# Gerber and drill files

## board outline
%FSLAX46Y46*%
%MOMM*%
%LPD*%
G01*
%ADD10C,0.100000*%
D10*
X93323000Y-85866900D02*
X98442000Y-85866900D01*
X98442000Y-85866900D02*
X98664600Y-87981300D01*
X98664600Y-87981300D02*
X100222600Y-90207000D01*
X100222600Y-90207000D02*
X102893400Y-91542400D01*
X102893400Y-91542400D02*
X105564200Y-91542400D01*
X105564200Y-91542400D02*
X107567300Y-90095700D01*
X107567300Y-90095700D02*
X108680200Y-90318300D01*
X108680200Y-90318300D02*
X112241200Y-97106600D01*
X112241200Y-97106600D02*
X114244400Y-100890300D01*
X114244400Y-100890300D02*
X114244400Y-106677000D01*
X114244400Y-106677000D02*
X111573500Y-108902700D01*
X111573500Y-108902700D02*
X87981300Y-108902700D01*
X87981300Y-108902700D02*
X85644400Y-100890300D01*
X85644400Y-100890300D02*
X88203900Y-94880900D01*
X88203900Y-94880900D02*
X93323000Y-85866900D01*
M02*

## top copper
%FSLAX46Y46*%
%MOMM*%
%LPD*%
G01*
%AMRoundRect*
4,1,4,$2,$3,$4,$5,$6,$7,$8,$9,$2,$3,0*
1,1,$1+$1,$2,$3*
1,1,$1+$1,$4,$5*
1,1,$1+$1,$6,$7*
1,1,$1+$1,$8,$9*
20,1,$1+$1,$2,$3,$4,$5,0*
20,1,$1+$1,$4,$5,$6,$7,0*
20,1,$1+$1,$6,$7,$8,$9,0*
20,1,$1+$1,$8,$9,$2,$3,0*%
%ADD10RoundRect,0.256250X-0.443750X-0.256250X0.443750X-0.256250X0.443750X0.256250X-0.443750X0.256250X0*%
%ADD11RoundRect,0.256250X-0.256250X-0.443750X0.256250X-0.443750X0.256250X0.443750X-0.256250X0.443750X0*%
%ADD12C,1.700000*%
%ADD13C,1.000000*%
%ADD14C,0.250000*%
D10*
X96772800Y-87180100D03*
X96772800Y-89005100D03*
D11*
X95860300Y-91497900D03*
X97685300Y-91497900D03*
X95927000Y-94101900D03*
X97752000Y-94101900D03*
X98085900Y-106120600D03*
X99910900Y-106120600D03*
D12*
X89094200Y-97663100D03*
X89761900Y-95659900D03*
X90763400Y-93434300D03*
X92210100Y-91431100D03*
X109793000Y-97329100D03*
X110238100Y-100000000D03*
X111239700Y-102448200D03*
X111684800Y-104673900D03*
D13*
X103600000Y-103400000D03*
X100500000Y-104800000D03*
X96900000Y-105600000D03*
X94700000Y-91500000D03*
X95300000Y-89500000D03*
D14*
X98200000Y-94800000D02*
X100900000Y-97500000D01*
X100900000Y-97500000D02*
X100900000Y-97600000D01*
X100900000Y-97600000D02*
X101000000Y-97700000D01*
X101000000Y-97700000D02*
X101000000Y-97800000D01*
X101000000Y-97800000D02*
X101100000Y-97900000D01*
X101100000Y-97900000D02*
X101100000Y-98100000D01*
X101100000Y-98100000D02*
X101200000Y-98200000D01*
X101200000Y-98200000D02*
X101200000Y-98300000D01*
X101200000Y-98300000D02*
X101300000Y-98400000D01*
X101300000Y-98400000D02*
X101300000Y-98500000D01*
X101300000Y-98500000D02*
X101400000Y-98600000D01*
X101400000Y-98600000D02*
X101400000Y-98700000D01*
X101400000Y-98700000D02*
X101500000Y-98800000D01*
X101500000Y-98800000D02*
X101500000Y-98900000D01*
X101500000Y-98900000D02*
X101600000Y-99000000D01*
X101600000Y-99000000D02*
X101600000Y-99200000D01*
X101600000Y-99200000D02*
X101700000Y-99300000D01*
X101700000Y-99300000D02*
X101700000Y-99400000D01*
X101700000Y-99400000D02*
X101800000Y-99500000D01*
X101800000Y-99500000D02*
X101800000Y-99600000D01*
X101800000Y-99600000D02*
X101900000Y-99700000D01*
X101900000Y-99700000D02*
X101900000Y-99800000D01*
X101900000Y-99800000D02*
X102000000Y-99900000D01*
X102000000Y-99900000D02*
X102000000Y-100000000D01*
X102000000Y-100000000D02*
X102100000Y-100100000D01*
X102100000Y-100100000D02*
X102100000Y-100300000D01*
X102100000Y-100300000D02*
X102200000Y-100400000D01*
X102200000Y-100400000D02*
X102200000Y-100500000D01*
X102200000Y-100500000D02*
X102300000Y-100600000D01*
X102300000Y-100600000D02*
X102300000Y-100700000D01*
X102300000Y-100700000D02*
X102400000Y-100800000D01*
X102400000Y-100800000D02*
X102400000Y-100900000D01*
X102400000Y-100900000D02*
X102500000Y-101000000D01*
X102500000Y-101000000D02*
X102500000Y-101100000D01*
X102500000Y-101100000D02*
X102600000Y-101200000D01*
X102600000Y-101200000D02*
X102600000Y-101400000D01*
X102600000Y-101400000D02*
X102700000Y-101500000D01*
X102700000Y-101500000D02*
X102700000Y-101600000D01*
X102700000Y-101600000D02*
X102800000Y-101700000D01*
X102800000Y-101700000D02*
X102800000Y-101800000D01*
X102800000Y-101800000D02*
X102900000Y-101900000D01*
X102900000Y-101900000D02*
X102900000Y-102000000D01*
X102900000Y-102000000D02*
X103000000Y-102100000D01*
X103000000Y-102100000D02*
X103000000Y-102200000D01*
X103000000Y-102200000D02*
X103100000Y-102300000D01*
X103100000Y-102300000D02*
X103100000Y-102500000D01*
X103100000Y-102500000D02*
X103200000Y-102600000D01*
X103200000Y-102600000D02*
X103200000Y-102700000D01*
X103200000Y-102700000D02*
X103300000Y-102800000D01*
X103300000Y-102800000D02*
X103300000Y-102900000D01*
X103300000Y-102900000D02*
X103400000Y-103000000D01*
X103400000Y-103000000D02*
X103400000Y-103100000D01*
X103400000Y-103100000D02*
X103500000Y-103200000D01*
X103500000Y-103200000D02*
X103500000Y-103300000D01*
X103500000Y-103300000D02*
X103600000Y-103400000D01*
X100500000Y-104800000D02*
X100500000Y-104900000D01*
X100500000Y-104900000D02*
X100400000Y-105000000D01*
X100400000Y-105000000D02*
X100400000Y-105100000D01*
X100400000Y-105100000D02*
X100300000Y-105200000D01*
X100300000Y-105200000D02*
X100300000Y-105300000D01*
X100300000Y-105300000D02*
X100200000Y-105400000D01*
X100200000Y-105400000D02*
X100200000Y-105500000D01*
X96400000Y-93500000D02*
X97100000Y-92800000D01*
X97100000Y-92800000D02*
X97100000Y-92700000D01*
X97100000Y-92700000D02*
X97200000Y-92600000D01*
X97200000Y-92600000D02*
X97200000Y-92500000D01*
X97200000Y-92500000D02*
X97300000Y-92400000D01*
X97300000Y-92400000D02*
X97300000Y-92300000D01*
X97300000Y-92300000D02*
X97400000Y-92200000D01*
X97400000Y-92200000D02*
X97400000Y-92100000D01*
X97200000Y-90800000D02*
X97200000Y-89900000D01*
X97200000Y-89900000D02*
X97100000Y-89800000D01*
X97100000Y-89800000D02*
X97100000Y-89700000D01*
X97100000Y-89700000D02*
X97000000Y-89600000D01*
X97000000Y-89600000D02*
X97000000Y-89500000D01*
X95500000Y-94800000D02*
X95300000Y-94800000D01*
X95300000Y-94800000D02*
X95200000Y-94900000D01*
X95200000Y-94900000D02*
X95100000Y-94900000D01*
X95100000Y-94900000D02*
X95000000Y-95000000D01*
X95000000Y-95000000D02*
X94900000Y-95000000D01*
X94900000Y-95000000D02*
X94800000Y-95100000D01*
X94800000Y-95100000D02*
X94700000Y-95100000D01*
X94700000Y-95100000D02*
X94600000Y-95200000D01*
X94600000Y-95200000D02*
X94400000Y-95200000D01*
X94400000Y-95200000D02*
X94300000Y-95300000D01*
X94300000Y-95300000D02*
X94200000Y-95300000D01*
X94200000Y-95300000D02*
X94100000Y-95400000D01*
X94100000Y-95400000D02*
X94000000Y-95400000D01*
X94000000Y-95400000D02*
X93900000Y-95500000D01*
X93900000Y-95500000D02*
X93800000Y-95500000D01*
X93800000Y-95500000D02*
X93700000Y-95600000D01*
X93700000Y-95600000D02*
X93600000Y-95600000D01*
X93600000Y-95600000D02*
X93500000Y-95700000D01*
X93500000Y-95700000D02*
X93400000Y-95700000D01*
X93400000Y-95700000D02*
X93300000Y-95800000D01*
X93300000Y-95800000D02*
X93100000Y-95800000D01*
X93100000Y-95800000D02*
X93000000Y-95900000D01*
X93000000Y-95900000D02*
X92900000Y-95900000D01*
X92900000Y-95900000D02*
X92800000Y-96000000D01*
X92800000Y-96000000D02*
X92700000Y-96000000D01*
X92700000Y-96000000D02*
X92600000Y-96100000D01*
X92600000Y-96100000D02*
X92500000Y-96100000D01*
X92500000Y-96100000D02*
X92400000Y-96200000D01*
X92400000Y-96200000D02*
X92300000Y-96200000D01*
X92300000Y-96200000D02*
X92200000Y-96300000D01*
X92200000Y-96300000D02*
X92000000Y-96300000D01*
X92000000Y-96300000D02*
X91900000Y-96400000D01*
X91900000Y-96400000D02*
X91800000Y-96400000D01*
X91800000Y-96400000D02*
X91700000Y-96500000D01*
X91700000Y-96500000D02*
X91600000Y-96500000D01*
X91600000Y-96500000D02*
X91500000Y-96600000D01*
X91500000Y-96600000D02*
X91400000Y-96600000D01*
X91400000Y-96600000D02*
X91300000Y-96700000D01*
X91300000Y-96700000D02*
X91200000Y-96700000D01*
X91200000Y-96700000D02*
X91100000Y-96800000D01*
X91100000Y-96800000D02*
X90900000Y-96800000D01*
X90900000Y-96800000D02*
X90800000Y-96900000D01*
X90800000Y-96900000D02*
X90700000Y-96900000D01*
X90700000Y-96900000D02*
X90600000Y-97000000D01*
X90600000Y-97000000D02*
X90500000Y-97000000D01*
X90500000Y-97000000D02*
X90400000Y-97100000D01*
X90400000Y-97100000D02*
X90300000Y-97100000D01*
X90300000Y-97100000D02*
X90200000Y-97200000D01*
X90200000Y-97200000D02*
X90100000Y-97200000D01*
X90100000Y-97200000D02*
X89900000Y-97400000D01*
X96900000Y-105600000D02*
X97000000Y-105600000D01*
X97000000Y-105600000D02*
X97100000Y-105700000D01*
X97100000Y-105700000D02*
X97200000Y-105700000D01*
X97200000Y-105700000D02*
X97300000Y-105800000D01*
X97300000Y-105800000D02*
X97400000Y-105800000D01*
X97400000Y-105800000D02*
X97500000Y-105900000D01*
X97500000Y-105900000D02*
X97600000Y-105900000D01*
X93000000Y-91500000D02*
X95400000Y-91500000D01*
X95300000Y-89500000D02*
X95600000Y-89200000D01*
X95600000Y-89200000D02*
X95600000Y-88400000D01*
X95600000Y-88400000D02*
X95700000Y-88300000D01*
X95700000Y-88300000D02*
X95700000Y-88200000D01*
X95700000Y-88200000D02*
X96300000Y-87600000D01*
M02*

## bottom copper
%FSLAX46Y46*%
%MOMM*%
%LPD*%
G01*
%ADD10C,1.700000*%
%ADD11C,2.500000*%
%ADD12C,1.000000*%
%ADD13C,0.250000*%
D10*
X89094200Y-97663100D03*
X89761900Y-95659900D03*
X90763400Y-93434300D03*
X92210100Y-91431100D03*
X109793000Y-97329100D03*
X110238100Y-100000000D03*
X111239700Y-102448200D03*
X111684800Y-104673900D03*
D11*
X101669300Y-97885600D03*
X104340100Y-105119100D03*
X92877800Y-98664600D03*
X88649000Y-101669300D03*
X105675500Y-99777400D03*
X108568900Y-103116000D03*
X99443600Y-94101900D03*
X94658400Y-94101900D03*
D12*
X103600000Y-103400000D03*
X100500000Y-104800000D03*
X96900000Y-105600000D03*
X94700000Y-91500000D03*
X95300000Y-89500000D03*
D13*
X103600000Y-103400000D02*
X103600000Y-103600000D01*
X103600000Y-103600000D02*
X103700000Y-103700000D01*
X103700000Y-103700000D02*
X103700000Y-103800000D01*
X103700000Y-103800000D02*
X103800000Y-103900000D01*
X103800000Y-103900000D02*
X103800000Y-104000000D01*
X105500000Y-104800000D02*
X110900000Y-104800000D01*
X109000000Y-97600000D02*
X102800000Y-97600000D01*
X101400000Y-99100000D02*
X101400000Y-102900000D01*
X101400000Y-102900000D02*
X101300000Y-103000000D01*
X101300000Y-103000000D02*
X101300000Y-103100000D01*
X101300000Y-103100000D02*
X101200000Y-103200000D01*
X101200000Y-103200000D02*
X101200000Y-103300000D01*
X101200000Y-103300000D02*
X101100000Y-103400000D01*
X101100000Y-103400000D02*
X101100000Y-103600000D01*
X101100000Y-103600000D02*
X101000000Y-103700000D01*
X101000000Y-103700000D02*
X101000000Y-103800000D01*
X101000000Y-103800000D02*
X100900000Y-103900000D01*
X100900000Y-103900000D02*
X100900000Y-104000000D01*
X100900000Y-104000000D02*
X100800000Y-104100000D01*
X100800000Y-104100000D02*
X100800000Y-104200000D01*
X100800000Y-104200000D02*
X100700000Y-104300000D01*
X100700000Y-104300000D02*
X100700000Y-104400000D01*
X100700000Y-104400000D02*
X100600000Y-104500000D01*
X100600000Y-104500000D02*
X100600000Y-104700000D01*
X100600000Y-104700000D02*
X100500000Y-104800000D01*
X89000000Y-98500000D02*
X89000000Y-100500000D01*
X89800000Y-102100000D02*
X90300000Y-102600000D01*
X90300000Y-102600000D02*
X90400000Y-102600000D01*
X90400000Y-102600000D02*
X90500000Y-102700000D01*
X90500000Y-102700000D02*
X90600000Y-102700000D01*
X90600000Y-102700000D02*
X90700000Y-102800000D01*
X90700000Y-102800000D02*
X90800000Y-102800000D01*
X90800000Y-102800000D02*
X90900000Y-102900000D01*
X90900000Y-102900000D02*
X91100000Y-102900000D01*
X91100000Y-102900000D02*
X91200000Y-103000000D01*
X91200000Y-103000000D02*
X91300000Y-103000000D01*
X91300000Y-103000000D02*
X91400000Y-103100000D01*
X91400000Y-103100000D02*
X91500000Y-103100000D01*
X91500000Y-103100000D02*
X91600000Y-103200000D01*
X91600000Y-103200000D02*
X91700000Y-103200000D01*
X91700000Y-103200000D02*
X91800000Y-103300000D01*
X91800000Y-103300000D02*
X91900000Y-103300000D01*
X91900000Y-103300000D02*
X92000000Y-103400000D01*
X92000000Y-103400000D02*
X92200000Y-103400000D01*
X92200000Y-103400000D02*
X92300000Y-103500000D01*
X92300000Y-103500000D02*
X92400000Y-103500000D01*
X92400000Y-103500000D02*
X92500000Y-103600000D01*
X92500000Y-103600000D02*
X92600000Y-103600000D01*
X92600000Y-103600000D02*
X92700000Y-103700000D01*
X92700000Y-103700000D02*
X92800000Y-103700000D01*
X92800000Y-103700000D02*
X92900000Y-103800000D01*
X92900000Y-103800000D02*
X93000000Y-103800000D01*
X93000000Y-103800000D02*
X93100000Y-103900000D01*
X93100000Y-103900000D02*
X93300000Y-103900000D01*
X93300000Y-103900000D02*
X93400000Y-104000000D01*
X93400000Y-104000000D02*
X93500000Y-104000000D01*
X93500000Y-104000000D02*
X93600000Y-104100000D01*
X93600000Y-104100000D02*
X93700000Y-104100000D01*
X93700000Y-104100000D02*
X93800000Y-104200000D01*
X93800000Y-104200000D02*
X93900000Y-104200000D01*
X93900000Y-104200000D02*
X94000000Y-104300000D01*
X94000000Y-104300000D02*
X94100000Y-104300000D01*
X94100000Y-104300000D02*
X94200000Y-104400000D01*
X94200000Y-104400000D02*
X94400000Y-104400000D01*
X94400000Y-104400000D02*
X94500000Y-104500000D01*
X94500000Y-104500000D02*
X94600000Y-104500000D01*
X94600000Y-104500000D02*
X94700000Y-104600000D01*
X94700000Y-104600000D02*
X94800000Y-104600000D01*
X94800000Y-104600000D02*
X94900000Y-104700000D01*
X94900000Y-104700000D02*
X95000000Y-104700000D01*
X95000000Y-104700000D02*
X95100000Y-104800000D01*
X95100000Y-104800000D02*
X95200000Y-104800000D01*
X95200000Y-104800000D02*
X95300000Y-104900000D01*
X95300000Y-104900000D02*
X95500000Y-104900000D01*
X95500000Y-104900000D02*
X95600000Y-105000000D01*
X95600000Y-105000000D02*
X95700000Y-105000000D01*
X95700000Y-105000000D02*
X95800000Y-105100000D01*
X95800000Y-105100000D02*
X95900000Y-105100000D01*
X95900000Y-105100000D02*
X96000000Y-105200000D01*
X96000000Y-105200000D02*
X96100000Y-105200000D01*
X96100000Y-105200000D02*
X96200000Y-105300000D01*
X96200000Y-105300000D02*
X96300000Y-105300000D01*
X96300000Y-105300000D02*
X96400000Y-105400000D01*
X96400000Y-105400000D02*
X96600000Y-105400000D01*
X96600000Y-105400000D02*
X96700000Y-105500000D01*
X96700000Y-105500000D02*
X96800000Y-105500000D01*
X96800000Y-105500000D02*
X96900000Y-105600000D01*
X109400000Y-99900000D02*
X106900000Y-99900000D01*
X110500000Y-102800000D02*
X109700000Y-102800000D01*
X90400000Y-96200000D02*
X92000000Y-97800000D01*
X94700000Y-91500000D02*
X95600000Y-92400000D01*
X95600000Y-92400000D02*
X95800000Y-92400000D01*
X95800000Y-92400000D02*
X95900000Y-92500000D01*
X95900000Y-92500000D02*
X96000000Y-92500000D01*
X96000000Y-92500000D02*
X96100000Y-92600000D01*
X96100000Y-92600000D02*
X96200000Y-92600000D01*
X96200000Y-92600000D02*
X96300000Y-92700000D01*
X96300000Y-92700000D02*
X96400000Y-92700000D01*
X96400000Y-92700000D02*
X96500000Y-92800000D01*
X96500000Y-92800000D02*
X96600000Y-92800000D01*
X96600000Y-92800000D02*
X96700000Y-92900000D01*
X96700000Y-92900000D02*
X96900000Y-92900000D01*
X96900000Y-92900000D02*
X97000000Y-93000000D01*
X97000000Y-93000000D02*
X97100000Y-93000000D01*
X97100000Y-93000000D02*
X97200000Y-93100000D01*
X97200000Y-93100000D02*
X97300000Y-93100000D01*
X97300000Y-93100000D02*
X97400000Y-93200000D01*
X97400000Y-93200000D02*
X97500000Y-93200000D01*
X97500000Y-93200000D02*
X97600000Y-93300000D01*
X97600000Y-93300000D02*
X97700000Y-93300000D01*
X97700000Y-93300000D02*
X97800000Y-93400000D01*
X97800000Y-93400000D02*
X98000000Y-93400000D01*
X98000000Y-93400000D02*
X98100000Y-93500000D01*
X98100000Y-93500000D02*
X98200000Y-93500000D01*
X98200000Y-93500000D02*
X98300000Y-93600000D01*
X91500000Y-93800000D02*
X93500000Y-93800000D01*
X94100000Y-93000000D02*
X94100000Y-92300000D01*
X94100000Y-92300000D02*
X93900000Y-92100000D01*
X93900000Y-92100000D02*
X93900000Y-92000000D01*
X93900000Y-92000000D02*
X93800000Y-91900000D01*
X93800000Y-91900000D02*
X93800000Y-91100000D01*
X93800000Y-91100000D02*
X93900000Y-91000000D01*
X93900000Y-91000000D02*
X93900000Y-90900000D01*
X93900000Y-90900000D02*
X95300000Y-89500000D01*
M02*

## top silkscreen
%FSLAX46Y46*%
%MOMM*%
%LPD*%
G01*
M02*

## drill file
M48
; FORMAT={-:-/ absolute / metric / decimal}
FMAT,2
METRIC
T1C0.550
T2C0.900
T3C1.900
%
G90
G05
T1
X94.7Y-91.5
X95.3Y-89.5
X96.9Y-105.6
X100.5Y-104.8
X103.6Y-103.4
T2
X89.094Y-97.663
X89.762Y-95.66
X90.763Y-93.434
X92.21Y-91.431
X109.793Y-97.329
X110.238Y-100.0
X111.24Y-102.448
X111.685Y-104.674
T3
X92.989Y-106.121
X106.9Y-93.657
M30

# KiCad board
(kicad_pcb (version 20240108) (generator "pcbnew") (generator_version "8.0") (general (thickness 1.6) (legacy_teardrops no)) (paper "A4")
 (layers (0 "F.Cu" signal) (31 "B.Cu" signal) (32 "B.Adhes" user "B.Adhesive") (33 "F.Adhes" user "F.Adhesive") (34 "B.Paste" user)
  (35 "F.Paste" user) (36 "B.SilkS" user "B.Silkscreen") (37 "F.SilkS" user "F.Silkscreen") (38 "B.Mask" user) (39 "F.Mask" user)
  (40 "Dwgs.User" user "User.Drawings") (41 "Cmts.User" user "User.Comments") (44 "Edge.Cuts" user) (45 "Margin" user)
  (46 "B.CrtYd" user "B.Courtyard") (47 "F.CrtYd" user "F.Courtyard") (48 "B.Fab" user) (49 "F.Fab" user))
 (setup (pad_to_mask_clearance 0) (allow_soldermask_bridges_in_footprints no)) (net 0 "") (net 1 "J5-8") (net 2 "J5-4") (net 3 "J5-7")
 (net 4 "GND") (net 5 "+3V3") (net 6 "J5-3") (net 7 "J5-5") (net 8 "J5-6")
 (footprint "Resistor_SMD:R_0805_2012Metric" (layer "F.Cu") (at 96.7728 88.0926)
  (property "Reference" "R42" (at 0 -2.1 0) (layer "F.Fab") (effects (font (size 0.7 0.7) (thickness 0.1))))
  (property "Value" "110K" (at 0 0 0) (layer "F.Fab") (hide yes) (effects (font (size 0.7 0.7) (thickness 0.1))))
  (pad "1" smd roundrect (at 0 -0.9125) (size 1.4 1.025) (layers "F.Cu" "F.Mask" "F.Paste") (roundrect_rratio 0.25) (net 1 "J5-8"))
  (pad "2" smd roundrect (at 0 0.9125) (size 1.4 1.025) (layers "F.Cu" "F.Mask" "F.Paste") (roundrect_rratio 0.25) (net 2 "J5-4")))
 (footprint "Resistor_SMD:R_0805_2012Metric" (layer "F.Cu") (at 96.7728 91.4979)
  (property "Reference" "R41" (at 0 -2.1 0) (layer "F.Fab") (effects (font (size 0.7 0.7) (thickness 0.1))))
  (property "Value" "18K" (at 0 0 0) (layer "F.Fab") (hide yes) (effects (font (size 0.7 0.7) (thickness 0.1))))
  (pad "1" smd roundrect (at -0.9125 0) (size 1.025 1.4) (layers "F.Cu" "F.Mask" "F.Paste") (roundrect_rratio 0.25) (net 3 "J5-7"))
  (pad "2" smd roundrect (at 0.9125 0) (size 1.025 1.4) (layers "F.Cu" "F.Mask" "F.Paste") (roundrect_rratio 0.25) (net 2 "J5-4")))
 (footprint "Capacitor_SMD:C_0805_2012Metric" (layer "F.Cu") (at 96.8395 94.1019)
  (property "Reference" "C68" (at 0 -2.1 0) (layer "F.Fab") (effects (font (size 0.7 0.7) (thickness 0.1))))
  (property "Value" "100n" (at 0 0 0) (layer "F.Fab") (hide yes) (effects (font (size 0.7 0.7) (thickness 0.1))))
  (pad "1" smd roundrect (at -0.9125 0) (size 1.025 1.4) (layers "F.Cu" "F.Mask" "F.Paste") (roundrect_rratio 0.25) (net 2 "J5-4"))
  (pad "2" smd roundrect (at 0.9125 0) (size 1.025 1.4) (layers "F.Cu" "F.Mask" "F.Paste") (roundrect_rratio 0.25) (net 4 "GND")))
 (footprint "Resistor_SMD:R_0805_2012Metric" (layer "F.Cu") (at 98.9984 106.1206)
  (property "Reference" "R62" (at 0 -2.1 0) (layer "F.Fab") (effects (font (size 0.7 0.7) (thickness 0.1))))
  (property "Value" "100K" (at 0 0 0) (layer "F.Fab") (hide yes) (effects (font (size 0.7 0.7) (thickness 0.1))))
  (pad "1" smd roundrect (at -0.9125 0) (size 1.025 1.4) (layers "F.Cu" "F.Mask" "F.Paste") (roundrect_rratio 0.25) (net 2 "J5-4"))
  (pad "2" smd roundrect (at 0.9125 0) (size 1.025 1.4) (layers "F.Cu" "F.Mask" "F.Paste") (roundrect_rratio 0.25) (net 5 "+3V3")))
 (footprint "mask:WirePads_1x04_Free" (layer "F.Cu") (at 90.4574 94.5471)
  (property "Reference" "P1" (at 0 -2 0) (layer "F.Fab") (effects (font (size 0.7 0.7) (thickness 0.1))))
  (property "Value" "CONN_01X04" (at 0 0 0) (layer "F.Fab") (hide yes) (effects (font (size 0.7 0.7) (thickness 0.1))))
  (pad "1" thru_hole circle (at -1.3632 3.116) (size 1.7 1.7) (drill 0.9) (layers "*.Cu" "*.Mask") (remove_unused_layers no) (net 2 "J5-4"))
  (pad "2" thru_hole circle (at -0.6955 1.1128) (size 1.7 1.7) (drill 0.9) (layers "*.Cu" "*.Mask") (remove_unused_layers no) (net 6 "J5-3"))
  (pad "3" thru_hole circle (at 0.306 -1.1128) (size 1.7 1.7) (drill 0.9) (layers "*.Cu" "*.Mask") (remove_unused_layers no) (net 1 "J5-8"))
  (pad "4" thru_hole circle (at 1.7527 -3.116) (size 1.7 1.7) (drill 0.9) (layers "*.Cu" "*.Mask") (remove_unused_layers no) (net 3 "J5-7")))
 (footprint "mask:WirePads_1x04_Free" (layer "F.Cu") (at 110.7389 101.1128)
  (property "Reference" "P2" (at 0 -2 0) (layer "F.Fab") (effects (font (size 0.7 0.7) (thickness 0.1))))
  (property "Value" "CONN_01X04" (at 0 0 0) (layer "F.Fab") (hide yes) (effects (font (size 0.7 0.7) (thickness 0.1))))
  (pad "1" thru_hole circle (at -0.9459 -3.7837) (size 1.7 1.7) (drill 0.9) (layers "*.Cu" "*.Mask") (remove_unused_layers no)
   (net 5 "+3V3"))
  (pad "2" thru_hole circle (at -0.5008 -1.1128) (size 1.7 1.7) (drill 0.9) (layers "*.Cu" "*.Mask") (remove_unused_layers no)
   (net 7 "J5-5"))
  (pad "3" thru_hole circle (at 0.5008 1.3354) (size 1.7 1.7) (drill 0.9) (layers "*.Cu" "*.Mask") (remove_unused_layers no) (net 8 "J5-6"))
  (pad "4" thru_hole circle (at 0.9459 3.5611) (size 1.7 1.7) (drill 0.9) (layers "*.Cu" "*.Mask") (remove_unused_layers no) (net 4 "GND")))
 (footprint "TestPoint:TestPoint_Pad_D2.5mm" (layer "B.Cu") (at 101.6693 97.8856)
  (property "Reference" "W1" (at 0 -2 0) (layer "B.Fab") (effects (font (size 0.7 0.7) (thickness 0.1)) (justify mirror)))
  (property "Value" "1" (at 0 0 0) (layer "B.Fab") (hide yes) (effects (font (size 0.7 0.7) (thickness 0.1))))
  (pad "1" smd circle (at 0 0) (size 2.5 2.5) (layers "B.Cu" "B.Mask") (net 5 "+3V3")))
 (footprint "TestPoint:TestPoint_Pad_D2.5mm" (layer "B.Cu") (at 104.3401 105.1191)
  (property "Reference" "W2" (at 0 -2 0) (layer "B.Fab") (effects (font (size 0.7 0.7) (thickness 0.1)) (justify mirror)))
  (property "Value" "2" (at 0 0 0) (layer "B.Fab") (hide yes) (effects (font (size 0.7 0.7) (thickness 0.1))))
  (pad "1" smd circle (at 0 0) (size 2.5 2.5) (layers "B.Cu" "B.Mask") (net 4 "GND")))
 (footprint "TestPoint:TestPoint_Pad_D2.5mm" (layer "B.Cu") (at 92.8778 98.6646)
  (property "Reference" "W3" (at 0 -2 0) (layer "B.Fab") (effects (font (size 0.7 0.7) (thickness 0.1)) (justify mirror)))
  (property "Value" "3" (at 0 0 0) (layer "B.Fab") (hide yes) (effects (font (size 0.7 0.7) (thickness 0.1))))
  (pad "1" smd circle (at 0 0) (size 2.5 2.5) (layers "B.Cu" "B.Mask") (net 6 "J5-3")))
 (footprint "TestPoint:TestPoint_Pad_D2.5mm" (layer "B.Cu") (at 88.649 101.6693)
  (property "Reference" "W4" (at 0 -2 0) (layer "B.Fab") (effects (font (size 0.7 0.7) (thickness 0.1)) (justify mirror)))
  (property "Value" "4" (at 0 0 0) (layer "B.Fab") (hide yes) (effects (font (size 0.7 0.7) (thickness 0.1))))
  (pad "1" smd circle (at 0 0) (size 2.5 2.5) (layers "B.Cu" "B.Mask") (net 2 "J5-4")))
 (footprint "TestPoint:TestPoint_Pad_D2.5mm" (layer "B.Cu") (at 105.6755 99.7774)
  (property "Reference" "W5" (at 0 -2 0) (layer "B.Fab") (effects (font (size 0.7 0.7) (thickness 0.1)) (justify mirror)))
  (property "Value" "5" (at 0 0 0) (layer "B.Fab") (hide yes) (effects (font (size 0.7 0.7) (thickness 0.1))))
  (pad "1" smd circle (at 0 0) (size 2.5 2.5) (layers "B.Cu" "B.Mask") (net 7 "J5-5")))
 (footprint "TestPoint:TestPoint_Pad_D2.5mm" (layer "B.Cu") (at 108.5689 103.116)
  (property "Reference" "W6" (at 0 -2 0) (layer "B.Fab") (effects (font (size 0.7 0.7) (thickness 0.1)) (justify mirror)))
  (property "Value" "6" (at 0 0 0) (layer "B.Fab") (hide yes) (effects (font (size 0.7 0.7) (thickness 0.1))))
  (pad "1" smd circle (at 0 0) (size 2.5 2.5) (layers "B.Cu" "B.Mask") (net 8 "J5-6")))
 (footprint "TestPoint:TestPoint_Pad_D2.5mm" (layer "B.Cu") (at 99.4436 94.1019)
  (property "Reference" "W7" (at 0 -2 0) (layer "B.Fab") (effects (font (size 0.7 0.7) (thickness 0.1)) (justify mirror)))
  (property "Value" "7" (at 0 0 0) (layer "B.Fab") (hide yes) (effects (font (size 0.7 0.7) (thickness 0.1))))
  (pad "1" smd circle (at 0 0) (size 2.5 2.5) (layers "B.Cu" "B.Mask") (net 3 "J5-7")))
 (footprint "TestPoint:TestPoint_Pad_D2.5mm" (layer "B.Cu") (at 94.6584 94.1019)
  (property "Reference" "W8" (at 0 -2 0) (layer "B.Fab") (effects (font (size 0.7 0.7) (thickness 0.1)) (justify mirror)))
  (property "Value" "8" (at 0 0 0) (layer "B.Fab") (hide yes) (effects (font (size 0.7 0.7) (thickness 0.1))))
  (pad "1" smd circle (at 0 0) (size 2.5 2.5) (layers "B.Cu" "B.Mask") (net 1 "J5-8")))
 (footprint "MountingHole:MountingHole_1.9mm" (layer "F.Cu") (at 92.9891 106.1206)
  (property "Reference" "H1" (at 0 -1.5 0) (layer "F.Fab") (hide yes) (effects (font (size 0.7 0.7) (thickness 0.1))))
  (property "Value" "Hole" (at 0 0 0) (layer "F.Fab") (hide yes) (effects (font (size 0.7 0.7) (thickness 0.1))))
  (pad "" np_thru_hole circle (at 0 0) (size 1.9 1.9) (drill 1.9) (layers "*.Cu" "*.Mask")))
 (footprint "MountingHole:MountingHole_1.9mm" (layer "F.Cu") (at 106.8996 93.6568)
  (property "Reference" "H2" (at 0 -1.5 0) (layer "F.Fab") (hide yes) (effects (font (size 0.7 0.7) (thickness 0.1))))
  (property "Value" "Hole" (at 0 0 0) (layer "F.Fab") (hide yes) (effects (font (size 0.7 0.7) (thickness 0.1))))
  (pad "" np_thru_hole circle (at 0 0) (size 1.9 1.9) (drill 1.9) (layers "*.Cu" "*.Mask")))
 (segment (start 98.2 94.8) (end 100.9 97.5) (width 0.25) (layer "F.Cu") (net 4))
 (segment (start 100.9 97.5) (end 100.9 97.6) (width 0.25) (layer "F.Cu") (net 4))
 (segment (start 100.9 97.6) (end 101 97.7) (width 0.25) (layer "F.Cu") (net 4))
 (segment (start 101 97.7) (end 101 97.8) (width 0.25) (layer "F.Cu") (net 4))
 (segment (start 101 97.8) (end 101.1 97.9) (width 0.25) (layer "F.Cu") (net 4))
 (segment (start 101.1 97.9) (end 101.1 98.1) (width 0.25) (layer "F.Cu") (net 4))
 (segment (start 101.1 98.1) (end 101.2 98.2) (width 0.25) (layer "F.Cu") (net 4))
 (segment (start 101.2 98.2) (end 101.2 98.3) (width 0.25) (layer "F.Cu") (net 4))
 (segment (start 101.2 98.3) (end 101.3 98.4) (width 0.25) (layer "F.Cu") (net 4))
 (segment (start 101.3 98.4) (end 101.3 98.5) (width 0.25) (layer "F.Cu") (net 4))
 (segment (start 101.3 98.5) (end 101.4 98.6) (width 0.25) (layer "F.Cu") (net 4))
 (segment (start 101.4 98.6) (end 101.4 98.7) (width 0.25) (layer "F.Cu") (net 4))
 (segment (start 101.4 98.7) (end 101.5 98.8) (width 0.25) (layer "F.Cu") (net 4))
 (segment (start 101.5 98.8) (end 101.5 98.9) (width 0.25) (layer "F.Cu") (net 4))
 (segment (start 101.5 98.9) (end 101.6 99) (width 0.25) (layer "F.Cu") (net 4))
 (segment (start 101.6 99) (end 101.6 99.2) (width 0.25) (layer "F.Cu") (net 4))
 (segment (start 101.6 99.2) (end 101.7 99.3) (width 0.25) (layer "F.Cu") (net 4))
 (segment (start 101.7 99.3) (end 101.7 99.4) (width 0.25) (layer "F.Cu") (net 4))
 (segment (start 101.7 99.4) (end 101.8 99.5) (width 0.25) (layer "F.Cu") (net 4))
 (segment (start 101.8 99.5) (end 101.8 99.6) (width 0.25) (layer "F.Cu") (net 4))
 (segment (start 101.8 99.6) (end 101.9 99.7) (width 0.25) (layer "F.Cu") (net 4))
 (segment (start 101.9 99.7) (end 101.9 99.8) (width 0.25) (layer "F.Cu") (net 4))
 (segment (start 101.9 99.8) (end 102 99.9) (width 0.25) (layer "F.Cu") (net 4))
 (segment (start 102 99.9) (end 102 100) (width 0.25) (layer "F.Cu") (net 4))
 (segment (start 102 100) (end 102.1 100.1) (width 0.25) (layer "F.Cu") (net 4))
 (segment (start 102.1 100.1) (end 102.1 100.3) (width 0.25) (layer "F.Cu") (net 4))
 (segment (start 102.1 100.3) (end 102.2 100.4) (width 0.25) (layer "F.Cu") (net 4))
 (segment (start 102.2 100.4) (end 102.2 100.5) (width 0.25) (layer "F.Cu") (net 4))
 (segment (start 102.2 100.5) (end 102.3 100.6) (width 0.25) (layer "F.Cu") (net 4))
 (segment (start 102.3 100.6) (end 102.3 100.7) (width 0.25) (layer "F.Cu") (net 4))
 (segment (start 102.3 100.7) (end 102.4 100.8) (width 0.25) (layer "F.Cu") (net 4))
 (segment (start 102.4 100.8) (end 102.4 100.9) (width 0.25) (layer "F.Cu") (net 4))
 (segment (start 102.4 100.9) (end 102.5 101) (width 0.25) (layer "F.Cu") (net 4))
 (segment (start 102.5 101) (end 102.5 101.1) (width 0.25) (layer "F.Cu") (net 4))
 (segment (start 102.5 101.1) (end 102.6 101.2) (width 0.25) (layer "F.Cu") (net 4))
 (segment (start 102.6 101.2) (end 102.6 101.4) (width 0.25) (layer "F.Cu") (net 4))
 (segment (start 102.6 101.4) (end 102.7 101.5) (width 0.25) (layer "F.Cu") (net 4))
 (segment (start 102.7 101.5) (end 102.7 101.6) (width 0.25) (layer "F.Cu") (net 4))
 (segment (start 102.7 101.6) (end 102.8 101.7) (width 0.25) (layer "F.Cu") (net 4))
 (segment (start 102.8 101.7) (end 102.8 101.8) (width 0.25) (layer "F.Cu") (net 4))
 (segment (start 102.8 101.8) (end 102.9 101.9) (width 0.25) (layer "F.Cu") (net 4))
 (segment (start 102.9 101.9) (end 102.9 102) (width 0.25) (layer "F.Cu") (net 4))
 (segment (start 102.9 102) (end 103 102.1) (width 0.25) (layer "F.Cu") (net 4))
 (segment (start 103 102.1) (end 103 102.2) (width 0.25) (layer "F.Cu") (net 4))
 (segment (start 103 102.2) (end 103.1 102.3) (width 0.25) (layer "F.Cu") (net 4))
 (segment (start 103.1 102.3) (end 103.1 102.5) (width 0.25) (layer "F.Cu") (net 4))
 (segment (start 103.1 102.5) (end 103.2 102.6) (width 0.25) (layer "F.Cu") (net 4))
 (segment (start 103.2 102.6) (end 103.2 102.7) (width 0.25) (layer "F.Cu") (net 4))
 (segment (start 103.2 102.7) (end 103.3 102.8) (width 0.25) (layer "F.Cu") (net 4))
 (segment (start 103.3 102.8) (end 103.3 102.9) (width 0.25) (layer "F.Cu") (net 4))
 (segment (start 103.3 102.9) (end 103.4 103) (width 0.25) (layer "F.Cu") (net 4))
 (segment (start 103.4 103) (end 103.4 103.1) (width 0.25) (layer "F.Cu") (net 4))
 (segment (start 103.4 103.1) (end 103.5 103.2) (width 0.25) (layer "F.Cu") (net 4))
 (segment (start 103.5 103.2) (end 103.5 103.3) (width 0.25) (layer "F.Cu") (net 4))
 (segment (start 103.5 103.3) (end 103.6 103.4) (width 0.25) (layer "F.Cu") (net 4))
 (segment (start 103.6 103.4) (end 103.6 103.6) (width 0.25) (layer "B.Cu") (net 4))
 (segment (start 103.6 103.6) (end 103.7 103.7) (width 0.25) (layer "B.Cu") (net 4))
 (segment (start 103.7 103.7) (end 103.7 103.8) (width 0.25) (layer "B.Cu") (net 4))
 (segment (start 103.7 103.8) (end 103.8 103.9) (width 0.25) (layer "B.Cu") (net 4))
 (segment (start 103.8 103.9) (end 103.8 104) (width 0.25) (layer "B.Cu") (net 4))
 (segment (start 105.5 104.8) (end 110.9 104.8) (width 0.25) (layer "B.Cu") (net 4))
 (via (at 103.6 103.4) (size 1) (drill 0.55) (layers "F.Cu" "B.Cu") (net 4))
 (segment (start 109 97.6) (end 102.8 97.6) (width 0.25) (layer "B.Cu") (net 5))
 (segment (start 101.4 99.1) (end 101.4 102.9) (width 0.25) (layer "B.Cu") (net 5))
 (segment (start 101.4 102.9) (end 101.3 103) (width 0.25) (layer "B.Cu") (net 5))
 (segment (start 101.3 103) (end 101.3 103.1) (width 0.25) (layer "B.Cu") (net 5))
 (segment (start 101.3 103.1) (end 101.2 103.2) (width 0.25) (layer "B.Cu") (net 5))
 (segment (start 101.2 103.2) (end 101.2 103.3) (width 0.25) (layer "B.Cu") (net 5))
 (segment (start 101.2 103.3) (end 101.1 103.4) (width 0.25) (layer "B.Cu") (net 5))
 (segment (start 101.1 103.4) (end 101.1 103.6) (width 0.25) (layer "B.Cu") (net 5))
 (segment (start 101.1 103.6) (end 101 103.7) (width 0.25) (layer "B.Cu") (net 5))
 (segment (start 101 103.7) (end 101 103.8) (width 0.25) (layer "B.Cu") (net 5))
 (segment (start 101 103.8) (end 100.9 103.9) (width 0.25) (layer "B.Cu") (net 5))
 (segment (start 100.9 103.9) (end 100.9 104) (width 0.25) (layer "B.Cu") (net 5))
 (segment (start 100.9 104) (end 100.8 104.1) (width 0.25) (layer "B.Cu") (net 5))
 (segment (start 100.8 104.1) (end 100.8 104.2) (width 0.25) (layer "B.Cu") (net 5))
 (segment (start 100.8 104.2) (end 100.7 104.3) (width 0.25) (layer "B.Cu") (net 5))
 (segment (start 100.7 104.3) (end 100.7 104.4) (width 0.25) (layer "B.Cu") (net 5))
 (segment (start 100.7 104.4) (end 100.6 104.5) (width 0.25) (layer "B.Cu") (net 5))
 (segment (start 100.6 104.5) (end 100.6 104.7) (width 0.25) (layer "B.Cu") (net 5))
 (segment (start 100.6 104.7) (end 100.5 104.8) (width 0.25) (layer "B.Cu") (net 5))
 (segment (start 100.5 104.8) (end 100.5 104.9) (width 0.25) (layer "F.Cu") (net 5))
 (segment (start 100.5 104.9) (end 100.4 105) (width 0.25) (layer "F.Cu") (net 5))
 (segment (start 100.4 105) (end 100.4 105.1) (width 0.25) (layer "F.Cu") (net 5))
 (segment (start 100.4 105.1) (end 100.3 105.2) (width 0.25) (layer "F.Cu") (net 5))
 (segment (start 100.3 105.2) (end 100.3 105.3) (width 0.25) (layer "F.Cu") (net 5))
 (segment (start 100.3 105.3) (end 100.2 105.4) (width 0.25) (layer "F.Cu") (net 5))
 (segment (start 100.2 105.4) (end 100.2 105.5) (width 0.25) (layer "F.Cu") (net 5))
 (via (at 100.5 104.8) (size 1) (drill 0.55) (layers "F.Cu" "B.Cu") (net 5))
 (segment (start 96.4 93.5) (end 97.1 92.8) (width 0.25) (layer "F.Cu") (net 2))
 (segment (start 97.1 92.8) (end 97.1 92.7) (width 0.25) (layer "F.Cu") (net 2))
 (segment (start 97.1 92.7) (end 97.2 92.6) (width 0.25) (layer "F.Cu") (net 2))
 (segment (start 97.2 92.6) (end 97.2 92.5) (width 0.25) (layer "F.Cu") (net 2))
 (segment (start 97.2 92.5) (end 97.3 92.4) (width 0.25) (layer "F.Cu") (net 2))
 (segment (start 97.3 92.4) (end 97.3 92.3) (width 0.25) (layer "F.Cu") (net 2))
 (segment (start 97.3 92.3) (end 97.4 92.2) (width 0.25) (layer "F.Cu") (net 2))
 (segment (start 97.4 92.2) (end 97.4 92.1) (width 0.25) (layer "F.Cu") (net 2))
 (segment (start 97.2 90.8) (end 97.2 89.9) (width 0.25) (layer "F.Cu") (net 2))
 (segment (start 97.2 89.9) (end 97.1 89.8) (width 0.25) (layer "F.Cu") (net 2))
 (segment (start 97.1 89.8) (end 97.1 89.7) (width 0.25) (layer "F.Cu") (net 2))
 (segment (start 97.1 89.7) (end 97 89.6) (width 0.25) (layer "F.Cu") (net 2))
 (segment (start 97 89.6) (end 97 89.5) (width 0.25) (layer "F.Cu") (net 2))
 (segment (start 95.5 94.8) (end 95.3 94.8) (width 0.25) (layer "F.Cu") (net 2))
 (segment (start 95.3 94.8) (end 95.2 94.9) (width 0.25) (layer "F.Cu") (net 2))
 (segment (start 95.2 94.9) (end 95.1 94.9) (width 0.25) (layer "F.Cu") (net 2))
 (segment (start 95.1 94.9) (end 95 95) (width 0.25) (layer "F.Cu") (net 2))
 (segment (start 95 95) (end 94.9 95) (width 0.25) (layer "F.Cu") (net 2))
 (segment (start 94.9 95) (end 94.8 95.1) (width 0.25) (layer "F.Cu") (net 2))
 (segment (start 94.8 95.1) (end 94.7 95.1) (width 0.25) (layer "F.Cu") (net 2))
 (segment (start 94.7 95.1) (end 94.6 95.2) (width 0.25) (layer "F.Cu") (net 2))
 (segment (start 94.6 95.2) (end 94.4 95.2) (width 0.25) (layer "F.Cu") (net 2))
 (segment (start 94.4 95.2) (end 94.3 95.3) (width 0.25) (layer "F.Cu") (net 2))
 (segment (start 94.3 95.3) (end 94.2 95.3) (width 0.25) (layer "F.Cu") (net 2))
 (segment (start 94.2 95.3) (end 94.1 95.4) (width 0.25) (layer "F.Cu") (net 2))
 (segment (start 94.1 95.4) (end 94 95.4) (width 0.25) (layer "F.Cu") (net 2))
 (segment (start 94 95.4) (end 93.9 95.5) (width 0.25) (layer "F.Cu") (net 2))
 (segment (start 93.9 95.5) (end 93.8 95.5) (width 0.25) (layer "F.Cu") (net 2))
 (segment (start 93.8 95.5) (end 93.7 95.6) (width 0.25) (layer "F.Cu") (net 2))
 (segment (start 93.7 95.6) (end 93.6 95.6) (width 0.25) (layer "F.Cu") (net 2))
 (segment (start 93.6 95.6) (end 93.5 95.7) (width 0.25) (layer "F.Cu") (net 2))
 (segment (start 93.5 95.7) (end 93.4 95.7) (width 0.25) (layer "F.Cu") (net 2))
 (segment (start 93.4 95.7) (end 93.3 95.8) (width 0.25) (layer "F.Cu") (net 2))
 (segment (start 93.3 95.8) (end 93.1 95.8) (width 0.25) (layer "F.Cu") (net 2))
 (segment (start 93.1 95.8) (end 93 95.9) (width 0.25) (layer "F.Cu") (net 2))
 (segment (start 93 95.9) (end 92.9 95.9) (width 0.25) (layer "F.Cu") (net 2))
 (segment (start 92.9 95.9) (end 92.8 96) (width 0.25) (layer "F.Cu") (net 2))
 (segment (start 92.8 96) (end 92.7 96) (width 0.25) (layer "F.Cu") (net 2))
 (segment (start 92.7 96) (end 92.6 96.1) (width 0.25) (layer "F.Cu") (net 2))
 (segment (start 92.6 96.1) (end 92.5 96.1) (width 0.25) (layer "F.Cu") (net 2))
 (segment (start 92.5 96.1) (end 92.4 96.2) (width 0.25) (layer "F.Cu") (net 2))
 (segment (start 92.4 96.2) (end 92.3 96.2) (width 0.25) (layer "F.Cu") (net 2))
 (segment (start 92.3 96.2) (end 92.2 96.3) (width 0.25) (layer "F.Cu") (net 2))
 (segment (start 92.2 96.3) (end 92 96.3) (width 0.25) (layer "F.Cu") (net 2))
 (segment (start 92 96.3) (end 91.9 96.4) (width 0.25) (layer "F.Cu") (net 2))
 (segment (start 91.9 96.4) (end 91.8 96.4) (width 0.25) (layer "F.Cu") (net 2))
 (segment (start 91.8 96.4) (end 91.7 96.5) (width 0.25) (layer "F.Cu") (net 2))
 (segment (start 91.7 96.5) (end 91.6 96.5) (width 0.25) (layer "F.Cu") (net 2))
 (segment (start 91.6 96.5) (end 91.5 96.6) (width 0.25) (layer "F.Cu") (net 2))
 (segment (start 91.5 96.6) (end 91.4 96.6) (width 0.25) (layer "F.Cu") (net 2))
 (segment (start 91.4 96.6) (end 91.3 96.7) (width 0.25) (layer "F.Cu") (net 2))
 (segment (start 91.3 96.7) (end 91.2 96.7) (width 0.25) (layer "F.Cu") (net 2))
 (segment (start 91.2 96.7) (end 91.1 96.8) (width 0.25) (layer "F.Cu") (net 2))
 (segment (start 91.1 96.8) (end 90.9 96.8) (width 0.25) (layer "F.Cu") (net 2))
 (segment (start 90.9 96.8) (end 90.8 96.9) (width 0.25) (layer "F.Cu") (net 2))
 (segment (start 90.8 96.9) (end 90.7 96.9) (width 0.25) (layer "F.Cu") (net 2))
 (segment (start 90.7 96.9) (end 90.6 97) (width 0.25) (layer "F.Cu") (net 2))
 (segment (start 90.6 97) (end 90.5 97) (width 0.25) (layer "F.Cu") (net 2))
 (segment (start 90.5 97) (end 90.4 97.1) (width 0.25) (layer "F.Cu") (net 2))
 (segment (start 90.4 97.1) (end 90.3 97.1) (width 0.25) (layer "F.Cu") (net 2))
 (segment (start 90.3 97.1) (end 90.2 97.2) (width 0.25) (layer "F.Cu") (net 2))
 (segment (start 90.2 97.2) (end 90.1 97.2) (width 0.25) (layer "F.Cu") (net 2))
 (segment (start 90.1 97.2) (end 89.9 97.4) (width 0.25) (layer "F.Cu") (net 2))
 (segment (start 89 98.5) (end 89 100.5) (width 0.25) (layer "B.Cu") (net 2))
 (segment (start 89.8 102.1) (end 90.3 102.6) (width 0.25) (layer "B.Cu") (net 2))
 (segment (start 90.3 102.6) (end 90.4 102.6) (width 0.25) (layer "B.Cu") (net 2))
 (segment (start 90.4 102.6) (end 90.5 102.7) (width 0.25) (layer "B.Cu") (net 2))
 (segment (start 90.5 102.7) (end 90.6 102.7) (width 0.25) (layer "B.Cu") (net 2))
 (segment (start 90.6 102.7) (end 90.7 102.8) (width 0.25) (layer "B.Cu") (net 2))
 (segment (start 90.7 102.8) (end 90.8 102.8) (width 0.25) (layer "B.Cu") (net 2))
 (segment (start 90.8 102.8) (end 90.9 102.9) (width 0.25) (layer "B.Cu") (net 2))
 (segment (start 90.9 102.9) (end 91.1 102.9) (width 0.25) (layer "B.Cu") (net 2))
 (segment (start 91.1 102.9) (end 91.2 103) (width 0.25) (layer "B.Cu") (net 2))
 (segment (start 91.2 103) (end 91.3 103) (width 0.25) (layer "B.Cu") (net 2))
 (segment (start 91.3 103) (end 91.4 103.1) (width 0.25) (layer "B.Cu") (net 2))
 (segment (start 91.4 103.1) (end 91.5 103.1) (width 0.25) (layer "B.Cu") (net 2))
 (segment (start 91.5 103.1) (end 91.6 103.2) (width 0.25) (layer "B.Cu") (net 2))
 (segment (start 91.6 103.2) (end 91.7 103.2) (width 0.25) (layer "B.Cu") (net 2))
 (segment (start 91.7 103.2) (end 91.8 103.3) (width 0.25) (layer "B.Cu") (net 2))
 (segment (start 91.8 103.3) (end 91.9 103.3) (width 0.25) (layer "B.Cu") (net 2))
 (segment (start 91.9 103.3) (end 92 103.4) (width 0.25) (layer "B.Cu") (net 2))
 (segment (start 92 103.4) (end 92.2 103.4) (width 0.25) (layer "B.Cu") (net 2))
 (segment (start 92.2 103.4) (end 92.3 103.5) (width 0.25) (layer "B.Cu") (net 2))
 (segment (start 92.3 103.5) (end 92.4 103.5) (width 0.25) (layer "B.Cu") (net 2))
 (segment (start 92.4 103.5) (end 92.5 103.6) (width 0.25) (layer "B.Cu") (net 2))
 (segment (start 92.5 103.6) (end 92.6 103.6) (width 0.25) (layer "B.Cu") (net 2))
 (segment (start 92.6 103.6) (end 92.7 103.7) (width 0.25) (layer "B.Cu") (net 2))
 (segment (start 92.7 103.7) (end 92.8 103.7) (width 0.25) (layer "B.Cu") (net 2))
 (segment (start 92.8 103.7) (end 92.9 103.8) (width 0.25) (layer "B.Cu") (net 2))
 (segment (start 92.9 103.8) (end 93 103.8) (width 0.25) (layer "B.Cu") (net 2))
 (segment (start 93 103.8) (end 93.1 103.9) (width 0.25) (layer "B.Cu") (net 2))
 (segment (start 93.1 103.9) (end 93.3 103.9) (width 0.25) (layer "B.Cu") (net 2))
 (segment (start 93.3 103.9) (end 93.4 104) (width 0.25) (layer "B.Cu") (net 2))
 (segment (start 93.4 104) (end 93.5 104) (width 0.25) (layer "B.Cu") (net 2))
 (segment (start 93.5 104) (end 93.6 104.1) (width 0.25) (layer "B.Cu") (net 2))
 (segment (start 93.6 104.1) (end 93.7 104.1) (width 0.25) (layer "B.Cu") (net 2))
 (segment (start 93.7 104.1) (end 93.8 104.2) (width 0.25) (layer "B.Cu") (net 2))
 (segment (start 93.8 104.2) (end 93.9 104.2) (width 0.25) (layer "B.Cu") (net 2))
 (segment (start 93.9 104.2) (end 94 104.3) (width 0.25) (layer "B.Cu") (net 2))
 (segment (start 94 104.3) (end 94.1 104.3) (width 0.25) (layer "B.Cu") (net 2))
 (segment (start 94.1 104.3) (end 94.2 104.4) (width 0.25) (layer "B.Cu") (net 2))
 (segment (start 94.2 104.4) (end 94.4 104.4) (width 0.25) (layer "B.Cu") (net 2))
 (segment (start 94.4 104.4) (end 94.5 104.5) (width 0.25) (layer "B.Cu") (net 2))
 (segment (start 94.5 104.5) (end 94.6 104.5) (width 0.25) (layer "B.Cu") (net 2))
 (segment (start 94.6 104.5) (end 94.7 104.6) (width 0.25) (layer "B.Cu") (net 2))
 (segment (start 94.7 104.6) (end 94.8 104.6) (width 0.25) (layer "B.Cu") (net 2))
 (segment (start 94.8 104.6) (end 94.9 104.7) (width 0.25) (layer "B.Cu") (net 2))
 (segment (start 94.9 104.7) (end 95 104.7) (width 0.25) (layer "B.Cu") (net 2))
 (segment (start 95 104.7) (end 95.1 104.8) (width 0.25) (layer "B.Cu") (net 2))
 (segment (start 95.1 104.8) (end 95.2 104.8) (width 0.25) (layer "B.Cu") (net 2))
 (segment (start 95.2 104.8) (end 95.3 104.9) (width 0.25) (layer "B.Cu") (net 2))
 (segment (start 95.3 104.9) (end 95.5 104.9) (width 0.25) (layer "B.Cu") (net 2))
 (segment (start 95.5 104.9) (end 95.6 105) (width 0.25) (layer "B.Cu") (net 2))
 (segment (start 95.6 105) (end 95.7 105) (width 0.25) (layer "B.Cu") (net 2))
 (segment (start 95.7 105) (end 95.8 105.1) (width 0.25) (layer "B.Cu") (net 2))
 (segment (start 95.8 105.1) (end 95.9 105.1) (width 0.25) (layer "B.Cu") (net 2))
 (segment (start 95.9 105.1) (end 96 105.2) (width 0.25) (layer "B.Cu") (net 2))
 (segment (start 96 105.2) (end 96.1 105.2) (width 0.25) (layer "B.Cu") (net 2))
 (segment (start 96.1 105.2) (end 96.2 105.3) (width 0.25) (layer "B.Cu") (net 2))
 (segment (start 96.2 105.3) (end 96.3 105.3) (width 0.25) (layer "B.Cu") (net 2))
 (segment (start 96.3 105.3) (end 96.4 105.4) (width 0.25) (layer "B.Cu") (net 2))
 (segment (start 96.4 105.4) (end 96.6 105.4) (width 0.25) (layer "B.Cu") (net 2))
 (segment (start 96.6 105.4) (end 96.7 105.5) (width 0.25) (layer "B.Cu") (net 2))
 (segment (start 96.7 105.5) (end 96.8 105.5) (width 0.25) (layer "B.Cu") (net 2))
 (segment (start 96.8 105.5) (end 96.9 105.6) (width 0.25) (layer "B.Cu") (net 2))
 (segment (start 96.9 105.6) (end 97 105.6) (width 0.25) (layer "F.Cu") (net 2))
 (segment (start 97 105.6) (end 97.1 105.7) (width 0.25) (layer "F.Cu") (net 2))
 (segment (start 97.1 105.7) (end 97.2 105.7) (width 0.25) (layer "F.Cu") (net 2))
 (segment (start 97.2 105.7) (end 97.3 105.8) (width 0.25) (layer "F.Cu") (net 2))
 (segment (start 97.3 105.8) (end 97.4 105.8) (width 0.25) (layer "F.Cu") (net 2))
 (segment (start 97.4 105.8) (end 97.5 105.9) (width 0.25) (layer "F.Cu") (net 2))
 (segment (start 97.5 105.9) (end 97.6 105.9) (width 0.25) (layer "F.Cu") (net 2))
 (via (at 96.9 105.6) (size 1) (drill 0.55) (layers "F.Cu" "B.Cu") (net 2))
 (segment (start 109.4 99.9) (end 106.9 99.9) (width 0.25) (layer "B.Cu") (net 7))
 (segment (start 110.5 102.8) (end 109.7 102.8) (width 0.25) (layer "B.Cu") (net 8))
 (segment (start 90.4 96.2) (end 92 97.8) (width 0.25) (layer "B.Cu") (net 6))
 (segment (start 93 91.5) (end 95.4 91.5) (width 0.25) (layer "F.Cu") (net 3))
 (segment (start 94.7 91.5) (end 95.6 92.4) (width 0.25) (layer "B.Cu") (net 3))
 (segment (start 95.6 92.4) (end 95.8 92.4) (width 0.25) (layer "B.Cu") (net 3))
 (segment (start 95.8 92.4) (end 95.9 92.5) (width 0.25) (layer "B.Cu") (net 3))
 (segment (start 95.9 92.5) (end 96 92.5) (width 0.25) (layer "B.Cu") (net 3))
 (segment (start 96 92.5) (end 96.1 92.6) (width 0.25) (layer "B.Cu") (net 3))
 (segment (start 96.1 92.6) (end 96.2 92.6) (width 0.25) (layer "B.Cu") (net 3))
 (segment (start 96.2 92.6) (end 96.3 92.7) (width 0.25) (layer "B.Cu") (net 3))
 (segment (start 96.3 92.7) (end 96.4 92.7) (width 0.25) (layer "B.Cu") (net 3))
 (segment (start 96.4 92.7) (end 96.5 92.8) (width 0.25) (layer "B.Cu") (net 3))
 (segment (start 96.5 92.8) (end 96.6 92.8) (width 0.25) (layer "B.Cu") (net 3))
 (segment (start 96.6 92.8) (end 96.7 92.9) (width 0.25) (layer "B.Cu") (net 3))
 (segment (start 96.7 92.9) (end 96.9 92.9) (width 0.25) (layer "B.Cu") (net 3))
 (segment (start 96.9 92.9) (end 97 93) (width 0.25) (layer "B.Cu") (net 3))
 (segment (start 97 93) (end 97.1 93) (width 0.25) (layer "B.Cu") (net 3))
 (segment (start 97.1 93) (end 97.2 93.1) (width 0.25) (layer "B.Cu") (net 3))
 (segment (start 97.2 93.1) (end 97.3 93.1) (width 0.25) (layer "B.Cu") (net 3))
 (segment (start 97.3 93.1) (end 97.4 93.2) (width 0.25) (layer "B.Cu") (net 3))
 (segment (start 97.4 93.2) (end 97.5 93.2) (width 0.25) (layer "B.Cu") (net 3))
 (segment (start 97.5 93.2) (end 97.6 93.3) (width 0.25) (layer "B.Cu") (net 3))
 (segment (start 97.6 93.3) (end 97.7 93.3) (width 0.25) (layer "B.Cu") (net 3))
 (segment (start 97.7 93.3) (end 97.8 93.4) (width 0.25) (layer "B.Cu") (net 3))
 (segment (start 97.8 93.4) (end 98 93.4) (width 0.25) (layer "B.Cu") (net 3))
 (segment (start 98 93.4) (end 98.1 93.5) (width 0.25) (layer "B.Cu") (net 3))
 (segment (start 98.1 93.5) (end 98.2 93.5) (width 0.25) (layer "B.Cu") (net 3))
 (segment (start 98.2 93.5) (end 98.3 93.6) (width 0.25) (layer "B.Cu") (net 3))
 (via (at 94.7 91.5) (size 1) (drill 0.55) (layers "F.Cu" "B.Cu") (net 3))
 (segment (start 91.5 93.8) (end 93.5 93.8) (width 0.25) (layer "B.Cu") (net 1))
 (segment (start 94.1 93) (end 94.1 92.3) (width 0.25) (layer "B.Cu") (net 1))
 (segment (start 94.1 92.3) (end 93.9 92.1) (width 0.25) (layer "B.Cu") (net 1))
 (segment (start 93.9 92.1) (end 93.9 92) (width 0.25) (layer "B.Cu") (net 1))
 (segment (start 93.9 92) (end 93.8 91.9) (width 0.25) (layer "B.Cu") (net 1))
 (segment (start 93.8 91.9) (end 93.8 91.1) (width 0.25) (layer "B.Cu") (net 1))
 (segment (start 93.8 91.1) (end 93.9 91) (width 0.25) (layer "B.Cu") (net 1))
 (segment (start 93.9 91) (end 93.9 90.9) (width 0.25) (layer "B.Cu") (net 1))
 (segment (start 93.9 90.9) (end 95.3 89.5) (width 0.25) (layer "B.Cu") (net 1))
 (segment (start 95.3 89.5) (end 95.6 89.2) (width 0.25) (layer "F.Cu") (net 1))
 (segment (start 95.6 89.2) (end 95.6 88.4) (width 0.25) (layer "F.Cu") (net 1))
 (segment (start 95.6 88.4) (end 95.7 88.3) (width 0.25) (layer "F.Cu") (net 1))
 (segment (start 95.7 88.3) (end 95.7 88.2) (width 0.25) (layer "F.Cu") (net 1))
 (segment (start 95.7 88.2) (end 96.3 87.6) (width 0.25) (layer "F.Cu") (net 1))
 (via (at 95.3 89.5) (size 1) (drill 0.55) (layers "F.Cu" "B.Cu") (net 1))
 (gr_line (start 93.323 85.8669) (end 98.442 85.8669) (stroke (width 0.1) (type default)) (layer "Edge.Cuts"))
 (gr_line (start 98.442 85.8669) (end 98.6646 87.9813) (stroke (width 0.1) (type default)) (layer "Edge.Cuts"))
 (gr_line (start 98.6646 87.9813) (end 100.2226 90.207) (stroke (width 0.1) (type default)) (layer "Edge.Cuts"))
 (gr_line (start 100.2226 90.207) (end 102.8934 91.5424) (stroke (width 0.1) (type default)) (layer "Edge.Cuts"))
 (gr_line (start 102.8934 91.5424) (end 105.5642 91.5424) (stroke (width 0.1) (type default)) (layer "Edge.Cuts"))
 (gr_line (start 105.5642 91.5424) (end 107.5673 90.0957) (stroke (width 0.1) (type default)) (layer "Edge.Cuts"))
 (gr_line (start 107.5673 90.0957) (end 108.6802 90.3183) (stroke (width 0.1) (type default)) (layer "Edge.Cuts"))
 (gr_line (start 108.6802 90.3183) (end 112.2412 97.1066) (stroke (width 0.1) (type default)) (layer "Edge.Cuts"))
 (gr_line (start 112.2412 97.1066) (end 114.2444 100.8903) (stroke (width 0.1) (type default)) (layer "Edge.Cuts"))
 (gr_line (start 114.2444 100.8903) (end 114.2444 106.677) (stroke (width 0.1) (type default)) (layer "Edge.Cuts"))
 (gr_line (start 114.2444 106.677) (end 111.5735 108.9027) (stroke (width 0.1) (type default)) (layer "Edge.Cuts"))
 (gr_line (start 111.5735 108.9027) (end 87.9813 108.9027) (stroke (width 0.1) (type default)) (layer "Edge.Cuts"))
 (gr_line (start 87.9813 108.9027) (end 85.6444 100.8903) (stroke (width 0.1) (type default)) (layer "Edge.Cuts"))
 (gr_line (start 85.6444 100.8903) (end 88.2039 94.8809) (stroke (width 0.1) (type default)) (layer "Edge.Cuts"))
 (gr_line (start 88.2039 94.8809) (end 93.323 85.8669) (stroke (width 0.1) (type default)) (layer "Edge.Cuts")))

